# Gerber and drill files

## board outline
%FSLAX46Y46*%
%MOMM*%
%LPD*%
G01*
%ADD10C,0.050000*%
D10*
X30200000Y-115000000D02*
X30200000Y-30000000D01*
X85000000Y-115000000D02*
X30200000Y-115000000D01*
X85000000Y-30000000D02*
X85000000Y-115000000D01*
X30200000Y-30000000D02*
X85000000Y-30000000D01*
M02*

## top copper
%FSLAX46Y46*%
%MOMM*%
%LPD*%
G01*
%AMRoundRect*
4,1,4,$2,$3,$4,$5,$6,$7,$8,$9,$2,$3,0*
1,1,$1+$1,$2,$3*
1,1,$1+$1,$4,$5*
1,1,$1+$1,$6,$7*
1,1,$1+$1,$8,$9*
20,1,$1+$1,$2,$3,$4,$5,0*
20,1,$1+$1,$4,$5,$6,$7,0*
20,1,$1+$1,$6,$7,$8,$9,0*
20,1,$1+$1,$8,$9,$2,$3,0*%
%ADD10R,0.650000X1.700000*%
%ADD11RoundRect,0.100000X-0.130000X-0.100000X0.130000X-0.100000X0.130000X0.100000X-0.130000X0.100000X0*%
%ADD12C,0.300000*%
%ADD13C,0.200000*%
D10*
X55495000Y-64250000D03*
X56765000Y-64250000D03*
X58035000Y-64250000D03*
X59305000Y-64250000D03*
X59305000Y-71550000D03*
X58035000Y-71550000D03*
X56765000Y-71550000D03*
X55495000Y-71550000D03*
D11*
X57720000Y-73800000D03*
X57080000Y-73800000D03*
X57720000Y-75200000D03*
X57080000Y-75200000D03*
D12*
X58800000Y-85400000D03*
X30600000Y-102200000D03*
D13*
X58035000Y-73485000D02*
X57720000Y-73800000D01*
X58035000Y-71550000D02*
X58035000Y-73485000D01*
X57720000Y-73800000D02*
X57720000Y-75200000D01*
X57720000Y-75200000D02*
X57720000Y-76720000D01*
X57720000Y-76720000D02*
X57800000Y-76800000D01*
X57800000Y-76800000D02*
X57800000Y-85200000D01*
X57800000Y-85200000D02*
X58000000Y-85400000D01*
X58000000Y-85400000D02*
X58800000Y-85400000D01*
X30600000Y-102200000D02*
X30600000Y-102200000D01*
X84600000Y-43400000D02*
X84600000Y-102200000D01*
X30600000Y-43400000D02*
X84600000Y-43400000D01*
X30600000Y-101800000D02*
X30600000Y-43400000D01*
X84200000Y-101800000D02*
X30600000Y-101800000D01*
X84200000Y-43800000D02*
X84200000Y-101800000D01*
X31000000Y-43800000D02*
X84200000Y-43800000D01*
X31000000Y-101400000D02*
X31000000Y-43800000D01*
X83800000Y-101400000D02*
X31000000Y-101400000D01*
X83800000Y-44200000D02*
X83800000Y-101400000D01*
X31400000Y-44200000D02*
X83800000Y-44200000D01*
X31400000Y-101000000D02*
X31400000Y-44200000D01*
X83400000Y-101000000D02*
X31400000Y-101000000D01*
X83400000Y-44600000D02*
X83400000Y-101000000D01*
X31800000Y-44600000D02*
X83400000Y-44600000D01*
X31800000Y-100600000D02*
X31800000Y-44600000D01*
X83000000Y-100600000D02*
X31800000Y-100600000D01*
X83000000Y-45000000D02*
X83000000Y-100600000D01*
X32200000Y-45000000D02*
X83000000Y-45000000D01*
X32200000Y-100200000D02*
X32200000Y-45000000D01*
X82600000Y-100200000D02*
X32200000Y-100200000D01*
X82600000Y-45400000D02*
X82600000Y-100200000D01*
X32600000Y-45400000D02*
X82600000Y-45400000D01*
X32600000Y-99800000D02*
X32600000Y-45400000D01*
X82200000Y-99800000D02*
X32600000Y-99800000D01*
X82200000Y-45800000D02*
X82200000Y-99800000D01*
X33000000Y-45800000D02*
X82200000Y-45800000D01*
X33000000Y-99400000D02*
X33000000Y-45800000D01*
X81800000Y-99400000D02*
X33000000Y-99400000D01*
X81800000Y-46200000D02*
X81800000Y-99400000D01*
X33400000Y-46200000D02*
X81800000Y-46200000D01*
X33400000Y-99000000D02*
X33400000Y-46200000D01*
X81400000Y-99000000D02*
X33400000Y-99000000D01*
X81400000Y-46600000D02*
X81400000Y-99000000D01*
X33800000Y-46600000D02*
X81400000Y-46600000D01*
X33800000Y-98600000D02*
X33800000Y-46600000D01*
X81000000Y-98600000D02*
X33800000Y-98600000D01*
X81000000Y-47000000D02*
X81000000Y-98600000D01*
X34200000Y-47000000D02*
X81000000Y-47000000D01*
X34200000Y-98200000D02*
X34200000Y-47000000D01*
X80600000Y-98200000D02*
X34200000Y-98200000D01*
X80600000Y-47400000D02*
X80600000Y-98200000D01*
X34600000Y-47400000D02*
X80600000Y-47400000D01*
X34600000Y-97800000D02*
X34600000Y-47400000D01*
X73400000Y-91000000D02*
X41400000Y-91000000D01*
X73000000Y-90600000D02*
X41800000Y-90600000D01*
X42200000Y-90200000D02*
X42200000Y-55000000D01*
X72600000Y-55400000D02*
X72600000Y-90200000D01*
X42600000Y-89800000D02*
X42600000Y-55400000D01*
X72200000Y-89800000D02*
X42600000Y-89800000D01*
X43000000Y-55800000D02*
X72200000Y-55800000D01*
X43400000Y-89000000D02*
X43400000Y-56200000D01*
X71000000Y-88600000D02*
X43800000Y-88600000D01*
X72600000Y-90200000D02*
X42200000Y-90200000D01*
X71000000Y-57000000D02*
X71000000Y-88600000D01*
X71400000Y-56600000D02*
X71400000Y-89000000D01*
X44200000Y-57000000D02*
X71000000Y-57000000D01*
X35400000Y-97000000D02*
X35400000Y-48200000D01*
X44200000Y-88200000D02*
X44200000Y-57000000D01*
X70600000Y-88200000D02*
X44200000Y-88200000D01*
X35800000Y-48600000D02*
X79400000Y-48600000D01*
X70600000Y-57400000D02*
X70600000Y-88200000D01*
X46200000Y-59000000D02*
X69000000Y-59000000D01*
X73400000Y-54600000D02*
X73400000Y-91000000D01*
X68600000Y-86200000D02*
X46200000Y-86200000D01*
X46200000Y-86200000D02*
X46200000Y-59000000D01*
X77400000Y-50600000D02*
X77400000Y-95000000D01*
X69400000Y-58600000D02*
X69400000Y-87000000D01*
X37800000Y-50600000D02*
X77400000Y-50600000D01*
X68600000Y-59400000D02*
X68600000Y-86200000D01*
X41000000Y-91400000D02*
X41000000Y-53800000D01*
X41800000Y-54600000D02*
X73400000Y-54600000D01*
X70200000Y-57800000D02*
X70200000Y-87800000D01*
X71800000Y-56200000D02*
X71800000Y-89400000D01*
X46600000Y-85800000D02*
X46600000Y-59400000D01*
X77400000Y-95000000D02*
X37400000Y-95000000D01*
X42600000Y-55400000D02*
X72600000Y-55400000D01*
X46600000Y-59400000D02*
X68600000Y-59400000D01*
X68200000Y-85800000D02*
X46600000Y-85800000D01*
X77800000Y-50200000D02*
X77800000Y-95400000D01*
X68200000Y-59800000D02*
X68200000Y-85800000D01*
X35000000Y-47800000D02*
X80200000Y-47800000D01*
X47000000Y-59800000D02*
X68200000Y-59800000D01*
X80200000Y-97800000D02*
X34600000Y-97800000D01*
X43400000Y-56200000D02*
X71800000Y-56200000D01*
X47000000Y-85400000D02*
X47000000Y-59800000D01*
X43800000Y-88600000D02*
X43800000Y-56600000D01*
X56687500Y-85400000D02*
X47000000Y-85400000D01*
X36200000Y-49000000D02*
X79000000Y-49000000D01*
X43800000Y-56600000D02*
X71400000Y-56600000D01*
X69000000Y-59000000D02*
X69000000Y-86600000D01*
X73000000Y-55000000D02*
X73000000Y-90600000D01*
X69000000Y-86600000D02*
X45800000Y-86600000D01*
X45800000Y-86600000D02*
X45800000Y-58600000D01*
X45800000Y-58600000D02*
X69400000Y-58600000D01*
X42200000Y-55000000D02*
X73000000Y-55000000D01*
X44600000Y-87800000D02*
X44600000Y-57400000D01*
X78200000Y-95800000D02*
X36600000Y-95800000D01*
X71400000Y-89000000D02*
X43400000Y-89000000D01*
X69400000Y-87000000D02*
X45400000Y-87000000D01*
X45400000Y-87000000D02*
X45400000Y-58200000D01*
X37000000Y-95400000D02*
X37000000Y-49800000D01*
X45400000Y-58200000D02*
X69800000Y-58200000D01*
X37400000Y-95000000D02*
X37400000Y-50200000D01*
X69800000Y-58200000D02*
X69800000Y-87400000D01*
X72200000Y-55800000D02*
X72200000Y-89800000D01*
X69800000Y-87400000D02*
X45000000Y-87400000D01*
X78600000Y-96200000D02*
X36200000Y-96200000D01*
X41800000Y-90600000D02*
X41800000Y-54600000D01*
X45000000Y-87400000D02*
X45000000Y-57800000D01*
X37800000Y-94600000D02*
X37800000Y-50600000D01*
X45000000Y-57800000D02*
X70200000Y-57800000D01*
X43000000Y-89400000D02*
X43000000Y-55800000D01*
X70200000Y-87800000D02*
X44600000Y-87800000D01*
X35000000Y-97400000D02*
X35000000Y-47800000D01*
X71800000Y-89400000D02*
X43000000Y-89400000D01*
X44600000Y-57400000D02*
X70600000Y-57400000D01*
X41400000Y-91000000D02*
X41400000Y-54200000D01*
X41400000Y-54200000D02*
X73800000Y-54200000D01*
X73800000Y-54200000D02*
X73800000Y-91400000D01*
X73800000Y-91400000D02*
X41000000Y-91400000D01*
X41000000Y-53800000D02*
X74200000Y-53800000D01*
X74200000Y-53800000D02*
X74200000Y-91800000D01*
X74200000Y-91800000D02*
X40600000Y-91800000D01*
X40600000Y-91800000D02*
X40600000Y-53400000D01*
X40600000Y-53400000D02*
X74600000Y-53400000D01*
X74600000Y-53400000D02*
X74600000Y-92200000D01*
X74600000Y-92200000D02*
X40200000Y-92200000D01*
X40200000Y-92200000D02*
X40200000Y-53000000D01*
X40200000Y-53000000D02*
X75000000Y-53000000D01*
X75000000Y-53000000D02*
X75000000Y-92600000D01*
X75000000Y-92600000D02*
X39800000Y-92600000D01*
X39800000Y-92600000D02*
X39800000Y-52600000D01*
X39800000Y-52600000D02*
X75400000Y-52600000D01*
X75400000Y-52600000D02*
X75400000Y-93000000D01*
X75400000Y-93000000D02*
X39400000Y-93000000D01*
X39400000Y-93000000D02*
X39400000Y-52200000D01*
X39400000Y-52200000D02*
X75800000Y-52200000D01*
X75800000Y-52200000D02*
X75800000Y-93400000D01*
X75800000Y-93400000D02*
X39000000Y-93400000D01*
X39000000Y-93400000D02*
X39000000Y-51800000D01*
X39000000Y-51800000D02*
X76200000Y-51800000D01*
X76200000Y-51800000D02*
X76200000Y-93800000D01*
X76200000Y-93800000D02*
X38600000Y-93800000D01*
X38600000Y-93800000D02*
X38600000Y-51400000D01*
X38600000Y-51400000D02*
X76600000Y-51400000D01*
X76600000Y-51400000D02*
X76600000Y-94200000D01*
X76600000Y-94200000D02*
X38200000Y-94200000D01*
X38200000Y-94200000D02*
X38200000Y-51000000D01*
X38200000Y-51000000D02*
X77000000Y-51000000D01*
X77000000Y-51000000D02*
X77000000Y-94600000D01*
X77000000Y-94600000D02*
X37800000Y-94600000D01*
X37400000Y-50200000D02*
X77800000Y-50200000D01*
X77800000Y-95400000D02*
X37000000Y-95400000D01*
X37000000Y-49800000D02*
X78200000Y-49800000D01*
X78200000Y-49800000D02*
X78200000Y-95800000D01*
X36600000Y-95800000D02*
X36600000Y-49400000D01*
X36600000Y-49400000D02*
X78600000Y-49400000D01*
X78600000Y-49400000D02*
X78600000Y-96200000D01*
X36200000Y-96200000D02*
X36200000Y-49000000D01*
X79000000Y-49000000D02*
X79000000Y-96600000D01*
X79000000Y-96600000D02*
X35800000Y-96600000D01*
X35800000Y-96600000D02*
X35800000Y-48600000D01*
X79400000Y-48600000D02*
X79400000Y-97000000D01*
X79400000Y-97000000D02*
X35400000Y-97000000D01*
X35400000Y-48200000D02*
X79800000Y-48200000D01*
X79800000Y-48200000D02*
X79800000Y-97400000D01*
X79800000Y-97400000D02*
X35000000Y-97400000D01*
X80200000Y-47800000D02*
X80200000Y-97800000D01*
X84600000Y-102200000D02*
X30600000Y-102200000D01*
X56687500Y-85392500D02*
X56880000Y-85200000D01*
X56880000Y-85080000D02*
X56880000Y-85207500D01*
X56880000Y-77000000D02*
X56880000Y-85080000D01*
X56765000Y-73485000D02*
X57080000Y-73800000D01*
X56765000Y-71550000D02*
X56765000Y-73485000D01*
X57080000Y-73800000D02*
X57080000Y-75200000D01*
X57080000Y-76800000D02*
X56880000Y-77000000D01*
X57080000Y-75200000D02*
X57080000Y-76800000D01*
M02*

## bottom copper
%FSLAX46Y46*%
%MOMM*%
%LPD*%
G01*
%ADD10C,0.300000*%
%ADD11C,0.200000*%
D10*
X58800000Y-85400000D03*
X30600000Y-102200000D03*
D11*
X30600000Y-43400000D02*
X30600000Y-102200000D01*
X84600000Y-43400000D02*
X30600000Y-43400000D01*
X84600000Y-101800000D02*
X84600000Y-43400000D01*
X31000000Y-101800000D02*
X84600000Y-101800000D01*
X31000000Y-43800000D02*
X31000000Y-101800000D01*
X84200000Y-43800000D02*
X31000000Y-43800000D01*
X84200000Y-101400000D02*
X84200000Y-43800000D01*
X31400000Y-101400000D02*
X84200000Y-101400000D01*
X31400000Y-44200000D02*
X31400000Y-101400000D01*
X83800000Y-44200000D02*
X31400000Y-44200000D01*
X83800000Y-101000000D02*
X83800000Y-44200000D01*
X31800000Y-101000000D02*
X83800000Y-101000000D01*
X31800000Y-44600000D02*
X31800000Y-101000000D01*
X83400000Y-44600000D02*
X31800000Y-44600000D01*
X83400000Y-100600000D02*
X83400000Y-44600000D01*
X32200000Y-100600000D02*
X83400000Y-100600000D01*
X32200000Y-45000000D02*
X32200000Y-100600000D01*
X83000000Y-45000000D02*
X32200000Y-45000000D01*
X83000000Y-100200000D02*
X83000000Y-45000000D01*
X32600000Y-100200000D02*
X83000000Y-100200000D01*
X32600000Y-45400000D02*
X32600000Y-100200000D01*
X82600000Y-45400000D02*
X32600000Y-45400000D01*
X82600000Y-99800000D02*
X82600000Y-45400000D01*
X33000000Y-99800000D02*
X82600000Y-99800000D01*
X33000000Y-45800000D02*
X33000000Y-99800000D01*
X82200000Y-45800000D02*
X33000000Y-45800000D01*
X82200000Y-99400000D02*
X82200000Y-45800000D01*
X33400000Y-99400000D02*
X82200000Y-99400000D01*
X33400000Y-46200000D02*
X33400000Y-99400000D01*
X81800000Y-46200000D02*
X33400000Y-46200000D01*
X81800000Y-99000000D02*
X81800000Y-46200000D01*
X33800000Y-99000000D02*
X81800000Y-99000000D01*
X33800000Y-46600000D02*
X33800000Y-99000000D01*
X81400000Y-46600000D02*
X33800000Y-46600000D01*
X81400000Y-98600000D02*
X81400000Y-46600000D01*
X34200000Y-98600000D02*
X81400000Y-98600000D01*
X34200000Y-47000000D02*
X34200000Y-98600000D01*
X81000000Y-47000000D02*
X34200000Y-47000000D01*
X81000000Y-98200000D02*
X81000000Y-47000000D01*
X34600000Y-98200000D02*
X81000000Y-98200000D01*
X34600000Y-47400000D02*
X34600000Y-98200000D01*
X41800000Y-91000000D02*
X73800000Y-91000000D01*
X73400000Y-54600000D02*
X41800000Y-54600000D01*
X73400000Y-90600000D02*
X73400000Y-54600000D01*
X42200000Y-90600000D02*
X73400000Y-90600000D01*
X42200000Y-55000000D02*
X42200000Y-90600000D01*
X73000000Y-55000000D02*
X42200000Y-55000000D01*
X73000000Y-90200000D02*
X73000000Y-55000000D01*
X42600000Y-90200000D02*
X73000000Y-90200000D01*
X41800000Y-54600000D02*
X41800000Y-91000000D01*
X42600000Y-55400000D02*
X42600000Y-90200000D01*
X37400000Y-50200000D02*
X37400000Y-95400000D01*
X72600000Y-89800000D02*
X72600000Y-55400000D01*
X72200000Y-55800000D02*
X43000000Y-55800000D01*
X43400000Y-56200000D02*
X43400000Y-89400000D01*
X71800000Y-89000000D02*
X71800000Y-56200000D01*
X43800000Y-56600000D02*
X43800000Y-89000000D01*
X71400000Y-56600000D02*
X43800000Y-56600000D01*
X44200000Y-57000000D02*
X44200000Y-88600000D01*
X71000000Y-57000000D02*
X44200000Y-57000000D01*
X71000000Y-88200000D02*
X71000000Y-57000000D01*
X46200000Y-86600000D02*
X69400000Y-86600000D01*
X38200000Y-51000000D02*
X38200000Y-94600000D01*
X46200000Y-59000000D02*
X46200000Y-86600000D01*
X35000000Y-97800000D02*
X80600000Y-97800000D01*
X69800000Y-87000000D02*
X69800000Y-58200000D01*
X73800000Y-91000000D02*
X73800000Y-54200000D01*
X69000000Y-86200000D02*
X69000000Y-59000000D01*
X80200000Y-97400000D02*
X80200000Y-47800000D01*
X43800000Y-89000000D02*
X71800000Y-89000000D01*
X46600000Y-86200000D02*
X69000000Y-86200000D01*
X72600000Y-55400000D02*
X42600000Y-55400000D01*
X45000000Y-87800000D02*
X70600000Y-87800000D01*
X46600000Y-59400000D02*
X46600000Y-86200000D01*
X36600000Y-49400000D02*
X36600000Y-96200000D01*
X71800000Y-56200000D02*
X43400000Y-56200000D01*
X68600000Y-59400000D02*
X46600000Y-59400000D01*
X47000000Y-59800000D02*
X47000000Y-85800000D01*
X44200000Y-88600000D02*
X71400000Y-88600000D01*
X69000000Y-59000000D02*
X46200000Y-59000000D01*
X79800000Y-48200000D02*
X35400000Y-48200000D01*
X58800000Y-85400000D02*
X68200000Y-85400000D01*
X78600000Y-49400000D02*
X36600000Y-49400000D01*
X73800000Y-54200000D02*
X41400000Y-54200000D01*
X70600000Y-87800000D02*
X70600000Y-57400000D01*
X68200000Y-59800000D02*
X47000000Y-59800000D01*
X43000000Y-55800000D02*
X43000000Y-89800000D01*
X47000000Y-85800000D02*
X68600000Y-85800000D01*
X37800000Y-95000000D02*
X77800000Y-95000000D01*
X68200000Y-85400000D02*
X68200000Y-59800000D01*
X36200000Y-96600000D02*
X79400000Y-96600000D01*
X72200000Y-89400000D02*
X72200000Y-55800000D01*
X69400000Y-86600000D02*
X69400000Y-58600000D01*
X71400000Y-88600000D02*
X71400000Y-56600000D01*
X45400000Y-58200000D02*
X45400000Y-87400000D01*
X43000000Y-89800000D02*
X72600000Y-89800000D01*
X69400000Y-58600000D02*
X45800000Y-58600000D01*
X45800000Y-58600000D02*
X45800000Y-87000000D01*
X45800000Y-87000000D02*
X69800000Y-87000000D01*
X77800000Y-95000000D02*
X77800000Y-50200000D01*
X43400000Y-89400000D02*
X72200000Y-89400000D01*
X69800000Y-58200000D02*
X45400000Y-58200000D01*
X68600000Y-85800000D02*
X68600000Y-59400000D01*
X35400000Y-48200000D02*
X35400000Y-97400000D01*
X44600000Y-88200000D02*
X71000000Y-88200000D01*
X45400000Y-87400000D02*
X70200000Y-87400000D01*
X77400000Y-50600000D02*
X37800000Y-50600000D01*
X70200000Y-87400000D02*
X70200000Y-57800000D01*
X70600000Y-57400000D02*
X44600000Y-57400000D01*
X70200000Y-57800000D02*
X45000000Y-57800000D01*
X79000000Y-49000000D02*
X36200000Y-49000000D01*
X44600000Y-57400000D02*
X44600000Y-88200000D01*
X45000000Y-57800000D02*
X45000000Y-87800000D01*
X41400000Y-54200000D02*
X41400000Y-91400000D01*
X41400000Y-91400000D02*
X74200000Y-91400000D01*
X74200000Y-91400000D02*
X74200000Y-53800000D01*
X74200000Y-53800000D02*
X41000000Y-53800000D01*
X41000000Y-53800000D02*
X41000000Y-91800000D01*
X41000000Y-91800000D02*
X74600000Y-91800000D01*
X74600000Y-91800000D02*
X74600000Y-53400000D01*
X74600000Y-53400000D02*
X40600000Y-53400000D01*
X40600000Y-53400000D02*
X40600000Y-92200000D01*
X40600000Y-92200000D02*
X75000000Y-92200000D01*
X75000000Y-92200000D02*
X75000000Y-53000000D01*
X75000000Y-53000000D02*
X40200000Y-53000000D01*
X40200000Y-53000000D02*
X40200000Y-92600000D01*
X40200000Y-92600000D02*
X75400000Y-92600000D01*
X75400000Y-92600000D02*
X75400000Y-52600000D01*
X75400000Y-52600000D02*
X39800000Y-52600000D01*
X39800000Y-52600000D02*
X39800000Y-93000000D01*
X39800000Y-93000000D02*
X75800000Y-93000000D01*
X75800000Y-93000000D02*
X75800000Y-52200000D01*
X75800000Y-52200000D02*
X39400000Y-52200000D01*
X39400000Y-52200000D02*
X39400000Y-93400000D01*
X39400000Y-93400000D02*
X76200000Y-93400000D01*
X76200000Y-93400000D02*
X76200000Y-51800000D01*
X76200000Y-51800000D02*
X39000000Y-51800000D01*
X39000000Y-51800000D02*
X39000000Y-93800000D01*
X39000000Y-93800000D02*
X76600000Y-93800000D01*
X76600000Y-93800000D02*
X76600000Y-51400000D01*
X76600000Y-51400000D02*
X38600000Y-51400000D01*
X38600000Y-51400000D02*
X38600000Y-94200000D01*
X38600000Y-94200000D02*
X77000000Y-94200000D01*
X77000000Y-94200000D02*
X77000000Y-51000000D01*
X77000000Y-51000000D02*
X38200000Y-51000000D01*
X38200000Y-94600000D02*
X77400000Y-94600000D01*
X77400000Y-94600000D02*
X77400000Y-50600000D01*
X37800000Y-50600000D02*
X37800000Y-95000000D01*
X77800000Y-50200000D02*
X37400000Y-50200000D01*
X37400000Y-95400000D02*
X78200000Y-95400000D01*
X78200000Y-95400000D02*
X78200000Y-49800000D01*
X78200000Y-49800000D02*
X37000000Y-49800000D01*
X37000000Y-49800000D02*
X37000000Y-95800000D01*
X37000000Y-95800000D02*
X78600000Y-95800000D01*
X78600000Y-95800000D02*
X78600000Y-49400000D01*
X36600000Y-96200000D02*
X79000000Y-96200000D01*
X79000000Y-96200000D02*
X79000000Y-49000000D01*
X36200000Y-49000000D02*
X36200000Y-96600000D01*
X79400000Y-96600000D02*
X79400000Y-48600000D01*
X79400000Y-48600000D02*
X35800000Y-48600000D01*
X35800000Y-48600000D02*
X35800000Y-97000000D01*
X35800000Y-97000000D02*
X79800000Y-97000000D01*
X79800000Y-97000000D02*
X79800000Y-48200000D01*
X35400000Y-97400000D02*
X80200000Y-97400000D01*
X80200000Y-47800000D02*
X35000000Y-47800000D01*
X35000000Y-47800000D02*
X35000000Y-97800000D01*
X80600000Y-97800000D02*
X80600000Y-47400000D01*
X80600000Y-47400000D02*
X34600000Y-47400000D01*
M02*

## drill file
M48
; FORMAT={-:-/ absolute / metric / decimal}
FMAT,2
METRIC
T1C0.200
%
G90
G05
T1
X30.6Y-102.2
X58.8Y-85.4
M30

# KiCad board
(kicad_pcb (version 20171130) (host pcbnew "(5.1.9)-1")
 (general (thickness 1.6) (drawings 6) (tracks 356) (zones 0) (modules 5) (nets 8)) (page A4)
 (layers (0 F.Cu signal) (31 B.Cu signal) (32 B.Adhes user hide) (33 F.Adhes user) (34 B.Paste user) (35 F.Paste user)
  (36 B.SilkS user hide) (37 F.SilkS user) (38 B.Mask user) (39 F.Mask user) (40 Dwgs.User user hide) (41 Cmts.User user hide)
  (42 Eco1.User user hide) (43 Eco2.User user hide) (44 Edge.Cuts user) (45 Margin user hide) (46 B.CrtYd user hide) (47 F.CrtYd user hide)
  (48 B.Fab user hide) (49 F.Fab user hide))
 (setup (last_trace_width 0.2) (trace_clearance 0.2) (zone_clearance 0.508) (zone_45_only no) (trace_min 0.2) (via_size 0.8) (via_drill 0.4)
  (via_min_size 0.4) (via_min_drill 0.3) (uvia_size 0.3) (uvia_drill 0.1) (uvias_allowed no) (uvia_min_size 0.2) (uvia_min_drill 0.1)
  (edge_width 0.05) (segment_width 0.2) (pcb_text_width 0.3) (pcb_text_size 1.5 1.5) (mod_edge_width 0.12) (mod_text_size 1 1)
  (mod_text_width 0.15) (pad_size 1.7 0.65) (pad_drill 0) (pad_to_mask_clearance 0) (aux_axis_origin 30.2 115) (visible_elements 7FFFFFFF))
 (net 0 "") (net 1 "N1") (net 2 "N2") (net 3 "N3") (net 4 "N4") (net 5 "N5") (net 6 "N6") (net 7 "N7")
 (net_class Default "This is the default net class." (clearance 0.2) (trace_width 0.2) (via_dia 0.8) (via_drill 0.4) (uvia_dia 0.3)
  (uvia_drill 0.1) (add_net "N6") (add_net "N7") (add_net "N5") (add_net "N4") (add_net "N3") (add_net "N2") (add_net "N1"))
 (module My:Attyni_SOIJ (layer F.Cu) (at 57.4 67.9 90)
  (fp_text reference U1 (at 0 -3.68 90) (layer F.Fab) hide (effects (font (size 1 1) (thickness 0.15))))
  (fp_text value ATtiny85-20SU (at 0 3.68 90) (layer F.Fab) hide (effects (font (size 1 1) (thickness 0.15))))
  (pad 8 smd rect (at 3.65 -1.905 90) (size 1.7 0.65) (layers F.Cu F.Paste F.Mask) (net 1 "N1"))
  (pad 7 smd rect (at 3.65 -0.635 90) (size 1.7 0.65) (layers F.Cu F.Paste F.Mask) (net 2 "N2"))
  (pad 6 smd rect (at 3.65 0.635 90) (size 1.7 0.65) (layers F.Cu F.Paste F.Mask) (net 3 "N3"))
  (pad 5 smd rect (at 3.65 1.905 90) (size 1.7 0.65) (layers F.Cu F.Paste F.Mask) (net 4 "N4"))
  (pad 4 smd rect (at -3.65 1.905 90) (size 1.7 0.65) (layers F.Cu F.Paste F.Mask) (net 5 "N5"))
  (pad 3 smd rect (at -3.65 0.635 90) (size 1.7 0.65) (layers F.Cu F.Paste F.Mask) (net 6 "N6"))
  (pad 2 smd rect (at -3.65 -0.635 90) (size 1.7 0.65) (layers F.Cu F.Paste F.Mask) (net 6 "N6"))
  (pad 1 smd rect (at -3.65 -1.905 90) (size 1.7 0.65) (layers F.Cu F.Paste F.Mask) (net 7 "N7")))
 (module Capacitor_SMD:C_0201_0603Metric (layer F.Cu) (at 57.4 73.8)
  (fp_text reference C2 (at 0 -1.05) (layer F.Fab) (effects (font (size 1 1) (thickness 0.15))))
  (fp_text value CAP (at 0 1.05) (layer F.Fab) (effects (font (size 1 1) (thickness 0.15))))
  (pad 2 smd roundrect (at 0.32 0) (size 0.46 0.4) (layers F.Cu F.Mask) (roundrect_rratio 0.25) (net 6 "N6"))
  (pad 1 smd roundrect (at -0.32 0) (size 0.46 0.4) (layers F.Cu F.Mask) (roundrect_rratio 0.25) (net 6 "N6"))
  (pad "" smd roundrect (at 0.345 0) (size 0.318 0.36) (layers F.Paste) (roundrect_rratio 0.25))
  (pad "" smd roundrect (at -0.345 0) (size 0.318 0.36) (layers F.Paste) (roundrect_rratio 0.25)))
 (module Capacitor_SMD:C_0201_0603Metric (layer F.Cu) (at 57.4 75.2)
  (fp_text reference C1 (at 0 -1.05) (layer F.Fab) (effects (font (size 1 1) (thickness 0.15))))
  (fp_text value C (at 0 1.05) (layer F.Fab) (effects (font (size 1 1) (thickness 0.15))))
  (pad 2 smd roundrect (at 0.32 0) (size 0.46 0.4) (layers F.Cu F.Mask) (roundrect_rratio 0.25) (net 6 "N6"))
  (pad 1 smd roundrect (at -0.32 0) (size 0.46 0.4) (layers F.Cu F.Mask) (roundrect_rratio 0.25) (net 6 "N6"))
  (pad "" smd roundrect (at 0.345 0) (size 0.318 0.36) (layers F.Paste) (roundrect_rratio 0.25))
  (pad "" smd roundrect (at -0.345 0) (size 0.318 0.36) (layers F.Paste) (roundrect_rratio 0.25)))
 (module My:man (layer F.Cu) (at 51.6 77.8)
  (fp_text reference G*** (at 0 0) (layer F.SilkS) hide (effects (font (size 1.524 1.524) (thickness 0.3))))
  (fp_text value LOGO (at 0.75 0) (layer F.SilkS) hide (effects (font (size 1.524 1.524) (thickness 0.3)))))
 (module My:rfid (layer B.Cu) (at 58.4 70.6 180)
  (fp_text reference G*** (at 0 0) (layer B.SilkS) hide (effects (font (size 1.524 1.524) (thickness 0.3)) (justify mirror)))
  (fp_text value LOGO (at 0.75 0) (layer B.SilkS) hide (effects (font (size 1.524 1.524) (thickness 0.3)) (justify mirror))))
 (gr_line (start 30.2 115) (end 30.2 30) (layer Edge.Cuts) (width 0.05))
 (gr_line (start 85 115) (end 30.2 115) (layer Edge.Cuts) (width 0.05))
 (gr_line (start 85 30) (end 85 115) (layer Edge.Cuts) (width 0.05))
 (gr_line (start 30.2 30) (end 85 30) (layer Edge.Cuts) (width 0.05))
 (segment (start 58.035 73.485) (end 57.72 73.8) (width 0.2) (layer F.Cu) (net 6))
 (segment (start 58.035 71.55) (end 58.035 73.485) (width 0.2) (layer F.Cu) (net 6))
 (segment (start 57.72 73.8) (end 57.72 75.2) (width 0.2) (layer F.Cu) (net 6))
 (segment (start 57.72 75.2) (end 57.72 76.72) (width 0.2) (layer F.Cu) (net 6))
 (segment (start 57.72 76.72) (end 57.8 76.8) (width 0.2) (layer F.Cu) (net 6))
 (segment (start 57.8 76.8) (end 57.8 85.2) (width 0.2) (layer F.Cu) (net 6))
 (segment (start 57.8 85.2) (end 58 85.4) (width 0.2) (layer F.Cu) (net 6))
 (segment (start 58 85.4) (end 58.8 85.4) (width 0.2) (layer F.Cu) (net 6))
 (via (at 58.8 85.4) (size 0.3) (drill 0.2) (layers F.Cu B.Cu) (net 6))
 (segment (start 30.6 102.2) (end 30.6 102.2) (width 0.2) (layer F.Cu) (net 6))
 (segment (start 84.6 43.4) (end 84.6 102.2) (width 0.2) (layer F.Cu) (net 6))
 (segment (start 30.6 43.4) (end 84.6 43.4) (width 0.2) (layer F.Cu) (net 6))
 (segment (start 30.6 101.8) (end 30.6 43.4) (width 0.2) (layer F.Cu) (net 6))
 (segment (start 84.2 101.8) (end 30.6 101.8) (width 0.2) (layer F.Cu) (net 6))
 (segment (start 84.2 43.8) (end 84.2 101.8) (width 0.2) (layer F.Cu) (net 6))
 (segment (start 31 43.8) (end 84.2 43.8) (width 0.2) (layer F.Cu) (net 6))
 (segment (start 31 101.4) (end 31 43.8) (width 0.2) (layer F.Cu) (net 6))
 (segment (start 83.8 101.4) (end 31 101.4) (width 0.2) (layer F.Cu) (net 6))
 (segment (start 83.8 44.2) (end 83.8 101.4) (width 0.2) (layer F.Cu) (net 6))
 (segment (start 31.4 44.2) (end 83.8 44.2) (width 0.2) (layer F.Cu) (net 6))
 (segment (start 31.4 101) (end 31.4 44.2) (width 0.2) (layer F.Cu) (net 6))
 (segment (start 83.4 101) (end 31.4 101) (width 0.2) (layer F.Cu) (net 6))
 (segment (start 83.4 44.6) (end 83.4 101) (width 0.2) (layer F.Cu) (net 6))
 (segment (start 31.8 44.6) (end 83.4 44.6) (width 0.2) (layer F.Cu) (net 6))
 (segment (start 31.8 100.6) (end 31.8 44.6) (width 0.2) (layer F.Cu) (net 6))
 (segment (start 83 100.6) (end 31.8 100.6) (width 0.2) (layer F.Cu) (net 6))
 (segment (start 83 45) (end 83 100.6) (width 0.2) (layer F.Cu) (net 6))
 (segment (start 32.2 45) (end 83 45) (width 0.2) (layer F.Cu) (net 6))
 (segment (start 32.2 100.2) (end 32.2 45) (width 0.2) (layer F.Cu) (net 6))
 (segment (start 82.6 100.2) (end 32.2 100.2) (width 0.2) (layer F.Cu) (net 6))
 (segment (start 82.6 45.4) (end 82.6 100.2) (width 0.2) (layer F.Cu) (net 6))
 (segment (start 32.6 45.4) (end 82.6 45.4) (width 0.2) (layer F.Cu) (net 6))
 (segment (start 32.6 99.8) (end 32.6 45.4) (width 0.2) (layer F.Cu) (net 6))
 (segment (start 82.2 99.8) (end 32.6 99.8) (width 0.2) (layer F.Cu) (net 6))
 (segment (start 82.2 45.8) (end 82.2 99.8) (width 0.2) (layer F.Cu) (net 6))
 (segment (start 33 45.8) (end 82.2 45.8) (width 0.2) (layer F.Cu) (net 6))
 (segment (start 33 99.4) (end 33 45.8) (width 0.2) (layer F.Cu) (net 6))
 (segment (start 81.8 99.4) (end 33 99.4) (width 0.2) (layer F.Cu) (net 6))
 (segment (start 81.8 46.2) (end 81.8 99.4) (width 0.2) (layer F.Cu) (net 6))
 (segment (start 33.4 46.2) (end 81.8 46.2) (width 0.2) (layer F.Cu) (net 6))
 (segment (start 33.4 99) (end 33.4 46.2) (width 0.2) (layer F.Cu) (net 6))
 (segment (start 81.4 99) (end 33.4 99) (width 0.2) (layer F.Cu) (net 6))
 (segment (start 81.4 46.6) (end 81.4 99) (width 0.2) (layer F.Cu) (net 6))
 (segment (start 33.8 46.6) (end 81.4 46.6) (width 0.2) (layer F.Cu) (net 6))
 (segment (start 33.8 98.6) (end 33.8 46.6) (width 0.2) (layer F.Cu) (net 6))
 (segment (start 81 98.6) (end 33.8 98.6) (width 0.2) (layer F.Cu) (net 6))
 (segment (start 81 47) (end 81 98.6) (width 0.2) (layer F.Cu) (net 6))
 (segment (start 34.2 47) (end 81 47) (width 0.2) (layer F.Cu) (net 6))
 (segment (start 34.2 98.2) (end 34.2 47) (width 0.2) (layer F.Cu) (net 6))
 (segment (start 80.6 98.2) (end 34.2 98.2) (width 0.2) (layer F.Cu) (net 6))
 (segment (start 80.6 47.4) (end 80.6 98.2) (width 0.2) (layer F.Cu) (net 6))
 (segment (start 34.6 47.4) (end 80.6 47.4) (width 0.2) (layer F.Cu) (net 6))
 (segment (start 34.6 97.8) (end 34.6 47.4) (width 0.2) (layer F.Cu) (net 6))
 (segment (start 73.4 91) (end 41.4 91) (width 0.2) (layer F.Cu) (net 6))
 (segment (start 73 90.6) (end 41.8 90.6) (width 0.2) (layer F.Cu) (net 6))
 (segment (start 42.2 90.2) (end 42.2 55) (width 0.2) (layer F.Cu) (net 6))
 (segment (start 72.6 55.4) (end 72.6 90.2) (width 0.2) (layer F.Cu) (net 6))
 (segment (start 42.6 89.8) (end 42.6 55.4) (width 0.2) (layer F.Cu) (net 6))
 (segment (start 72.2 89.8) (end 42.6 89.8) (width 0.2) (layer F.Cu) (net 6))
 (segment (start 43 55.8) (end 72.2 55.8) (width 0.2) (layer F.Cu) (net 6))
 (segment (start 43.4 89) (end 43.4 56.2) (width 0.2) (layer F.Cu) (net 6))
 (segment (start 71 88.6) (end 43.8 88.6) (width 0.2) (layer F.Cu) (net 6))
 (segment (start 72.6 90.2) (end 42.2 90.2) (width 0.2) (layer F.Cu) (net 6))
 (segment (start 71 57) (end 71 88.6) (width 0.2) (layer F.Cu) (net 6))
 (segment (start 71.4 56.6) (end 71.4 89) (width 0.2) (layer F.Cu) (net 6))
 (segment (start 44.2 57) (end 71 57) (width 0.2) (layer F.Cu) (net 6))
 (segment (start 35.4 97) (end 35.4 48.2) (width 0.2) (layer F.Cu) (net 6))
 (segment (start 44.2 88.2) (end 44.2 57) (width 0.2) (layer F.Cu) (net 6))
 (segment (start 70.6 88.2) (end 44.2 88.2) (width 0.2) (layer F.Cu) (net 6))
 (segment (start 35.8 48.6) (end 79.4 48.6) (width 0.2) (layer F.Cu) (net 6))
 (segment (start 70.6 57.4) (end 70.6 88.2) (width 0.2) (layer F.Cu) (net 6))
 (segment (start 46.2 59) (end 69 59) (width 0.2) (layer F.Cu) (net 6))
 (segment (start 73.4 54.6) (end 73.4 91) (width 0.2) (layer F.Cu) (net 6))
 (segment (start 68.6 86.2) (end 46.2 86.2) (width 0.2) (layer F.Cu) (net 6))
 (segment (start 46.2 86.2) (end 46.2 59) (width 0.2) (layer F.Cu) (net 6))
 (segment (start 77.4 50.6) (end 77.4 95) (width 0.2) (layer F.Cu) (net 6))
 (segment (start 69.4 58.6) (end 69.4 87) (width 0.2) (layer F.Cu) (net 6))
 (segment (start 37.8 50.6) (end 77.4 50.6) (width 0.2) (layer F.Cu) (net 6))
 (segment (start 68.6 59.4) (end 68.6 86.2) (width 0.2) (layer F.Cu) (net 6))
 (segment (start 41 91.4) (end 41 53.8) (width 0.2) (layer F.Cu) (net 6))
 (segment (start 41.8 54.6) (end 73.4 54.6) (width 0.2) (layer F.Cu) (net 6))
 (segment (start 70.2 57.8) (end 70.2 87.8) (width 0.2) (layer F.Cu) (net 6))
 (segment (start 71.8 56.2) (end 71.8 89.4) (width 0.2) (layer F.Cu) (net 6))
 (segment (start 46.6 85.8) (end 46.6 59.4) (width 0.2) (layer F.Cu) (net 6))
 (segment (start 77.4 95) (end 37.4 95) (width 0.2) (layer F.Cu) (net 6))
 (segment (start 42.6 55.4) (end 72.6 55.4) (width 0.2) (layer F.Cu) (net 6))
 (segment (start 46.6 59.4) (end 68.6 59.4) (width 0.2) (layer F.Cu) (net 6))
 (segment (start 68.2 85.8) (end 46.6 85.8) (width 0.2) (layer F.Cu) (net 6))
 (segment (start 77.8 50.2) (end 77.8 95.4) (width 0.2) (layer F.Cu) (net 6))
 (segment (start 68.2 59.8) (end 68.2 85.8) (width 0.2) (layer F.Cu) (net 6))
 (segment (start 35 47.8) (end 80.2 47.8) (width 0.2) (layer F.Cu) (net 6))
 (segment (start 47 59.8) (end 68.2 59.8) (width 0.2) (layer F.Cu) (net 6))
 (segment (start 80.2 97.8) (end 34.6 97.8) (width 0.2) (layer F.Cu) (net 6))
 (segment (start 43.4 56.2) (end 71.8 56.2) (width 0.2) (layer F.Cu) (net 6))
 (segment (start 47 85.4) (end 47 59.8) (width 0.2) (layer F.Cu) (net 6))
 (segment (start 43.8 88.6) (end 43.8 56.6) (width 0.2) (layer F.Cu) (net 6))
 (segment (start 56.6875 85.4) (end 47 85.4) (width 0.2) (layer F.Cu) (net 6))
 (segment (start 36.2 49) (end 79 49) (width 0.2) (layer F.Cu) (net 6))
 (segment (start 43.8 56.6) (end 71.4 56.6) (width 0.2) (layer F.Cu) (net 6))
 (segment (start 69 59) (end 69 86.6) (width 0.2) (layer F.Cu) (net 6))
 (segment (start 73 55) (end 73 90.6) (width 0.2) (layer F.Cu) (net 6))
 (segment (start 69 86.6) (end 45.8 86.6) (width 0.2) (layer F.Cu) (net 6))
 (segment (start 45.8 86.6) (end 45.8 58.6) (width 0.2) (layer F.Cu) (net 6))
 (segment (start 45.8 58.6) (end 69.4 58.6) (width 0.2) (layer F.Cu) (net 6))
 (segment (start 42.2 55) (end 73 55) (width 0.2) (layer F.Cu) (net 6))
 (segment (start 44.6 87.8) (end 44.6 57.4) (width 0.2) (layer F.Cu) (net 6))
 (segment (start 78.2 95.8) (end 36.6 95.8) (width 0.2) (layer F.Cu) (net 6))
 (segment (start 71.4 89) (end 43.4 89) (width 0.2) (layer F.Cu) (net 6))
 (segment (start 69.4 87) (end 45.4 87) (width 0.2) (layer F.Cu) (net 6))
 (segment (start 45.4 87) (end 45.4 58.2) (width 0.2) (layer F.Cu) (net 6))
 (segment (start 37 95.4) (end 37 49.8) (width 0.2) (layer F.Cu) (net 6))
 (segment (start 45.4 58.2) (end 69.8 58.2) (width 0.2) (layer F.Cu) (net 6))
 (segment (start 37.4 95) (end 37.4 50.2) (width 0.2) (layer F.Cu) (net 6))
 (segment (start 69.8 58.2) (end 69.8 87.4) (width 0.2) (layer F.Cu) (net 6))
 (segment (start 72.2 55.8) (end 72.2 89.8) (width 0.2) (layer F.Cu) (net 6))
 (segment (start 69.8 87.4) (end 45 87.4) (width 0.2) (layer F.Cu) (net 6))
 (segment (start 78.6 96.2) (end 36.2 96.2) (width 0.2) (layer F.Cu) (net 6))
 (segment (start 41.8 90.6) (end 41.8 54.6) (width 0.2) (layer F.Cu) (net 6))
 (segment (start 45 87.4) (end 45 57.8) (width 0.2) (layer F.Cu) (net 6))
 (segment (start 37.8 94.6) (end 37.8 50.6) (width 0.2) (layer F.Cu) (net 6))
 (segment (start 45 57.8) (end 70.2 57.8) (width 0.2) (layer F.Cu) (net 6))
 (segment (start 43 89.4) (end 43 55.8) (width 0.2) (layer F.Cu) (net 6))
 (segment (start 70.2 87.8) (end 44.6 87.8) (width 0.2) (layer F.Cu) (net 6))
 (segment (start 35 97.4) (end 35 47.8) (width 0.2) (layer F.Cu) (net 6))
 (segment (start 71.8 89.4) (end 43 89.4) (width 0.2) (layer F.Cu) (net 6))
 (segment (start 44.6 57.4) (end 70.6 57.4) (width 0.2) (layer F.Cu) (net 6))
 (segment (start 41.4 91) (end 41.4 54.2) (width 0.2) (layer F.Cu) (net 6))
 (segment (start 41.4 54.2) (end 73.8 54.2) (width 0.2) (layer F.Cu) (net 6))
 (segment (start 73.8 54.2) (end 73.8 91.4) (width 0.2) (layer F.Cu) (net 6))
 (segment (start 73.8 91.4) (end 41 91.4) (width 0.2) (layer F.Cu) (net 6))
 (segment (start 41 53.8) (end 74.2 53.8) (width 0.2) (layer F.Cu) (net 6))
 (segment (start 74.2 53.8) (end 74.2 91.8) (width 0.2) (layer F.Cu) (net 6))
 (segment (start 74.2 91.8) (end 40.6 91.8) (width 0.2) (layer F.Cu) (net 6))
 (segment (start 40.6 91.8) (end 40.6 53.4) (width 0.2) (layer F.Cu) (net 6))
 (segment (start 40.6 53.4) (end 74.6 53.4) (width 0.2) (layer F.Cu) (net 6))
 (segment (start 74.6 53.4) (end 74.6 92.2) (width 0.2) (layer F.Cu) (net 6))
 (segment (start 74.6 92.2) (end 40.2 92.2) (width 0.2) (layer F.Cu) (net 6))
 (segment (start 40.2 92.2) (end 40.2 53) (width 0.2) (layer F.Cu) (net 6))
 (segment (start 40.2 53) (end 75 53) (width 0.2) (layer F.Cu) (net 6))
 (segment (start 75 53) (end 75 92.6) (width 0.2) (layer F.Cu) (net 6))
 (segment (start 75 92.6) (end 39.8 92.6) (width 0.2) (layer F.Cu) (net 6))
 (segment (start 39.8 92.6) (end 39.8 52.6) (width 0.2) (layer F.Cu) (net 6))
 (segment (start 39.8 52.6) (end 75.4 52.6) (width 0.2) (layer F.Cu) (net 6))
 (segment (start 75.4 52.6) (end 75.4 93) (width 0.2) (layer F.Cu) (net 6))
 (segment (start 75.4 93) (end 39.4 93) (width 0.2) (layer F.Cu) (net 6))
 (segment (start 39.4 93) (end 39.4 52.2) (width 0.2) (layer F.Cu) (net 6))
 (segment (start 39.4 52.2) (end 75.8 52.2) (width 0.2) (layer F.Cu) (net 6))
 (segment (start 75.8 52.2) (end 75.8 93.4) (width 0.2) (layer F.Cu) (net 6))
 (segment (start 75.8 93.4) (end 39 93.4) (width 0.2) (layer F.Cu) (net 6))
 (segment (start 39 93.4) (end 39 51.8) (width 0.2) (layer F.Cu) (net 6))
 (segment (start 39 51.8) (end 76.2 51.8) (width 0.2) (layer F.Cu) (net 6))
 (segment (start 76.2 51.8) (end 76.2 93.8) (width 0.2) (layer F.Cu) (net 6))
 (segment (start 76.2 93.8) (end 38.6 93.8) (width 0.2) (layer F.Cu) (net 6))
 (segment (start 38.6 93.8) (end 38.6 51.4) (width 0.2) (layer F.Cu) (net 6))
 (segment (start 38.6 51.4) (end 76.6 51.4) (width 0.2) (layer F.Cu) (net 6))
 (segment (start 76.6 51.4) (end 76.6 94.2) (width 0.2) (layer F.Cu) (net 6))
 (segment (start 76.6 94.2) (end 38.2 94.2) (width 0.2) (layer F.Cu) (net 6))
 (segment (start 38.2 94.2) (end 38.2 51) (width 0.2) (layer F.Cu) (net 6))
 (segment (start 38.2 51) (end 77 51) (width 0.2) (layer F.Cu) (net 6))
 (segment (start 77 51) (end 77 94.6) (width 0.2) (layer F.Cu) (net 6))
 (segment (start 77 94.6) (end 37.8 94.6) (width 0.2) (layer F.Cu) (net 6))
 (segment (start 37.4 50.2) (end 77.8 50.2) (width 0.2) (layer F.Cu) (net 6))
 (segment (start 77.8 95.4) (end 37 95.4) (width 0.2) (layer F.Cu) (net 6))
 (segment (start 37 49.8) (end 78.2 49.8) (width 0.2) (layer F.Cu) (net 6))
 (segment (start 78.2 49.8) (end 78.2 95.8) (width 0.2) (layer F.Cu) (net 6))
 (segment (start 36.6 95.8) (end 36.6 49.4) (width 0.2) (layer F.Cu) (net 6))
 (segment (start 36.6 49.4) (end 78.6 49.4) (width 0.2) (layer F.Cu) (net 6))
 (segment (start 78.6 49.4) (end 78.6 96.2) (width 0.2) (layer F.Cu) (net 6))
 (segment (start 36.2 96.2) (end 36.2 49) (width 0.2) (layer F.Cu) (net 6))
 (segment (start 79 49) (end 79 96.6) (width 0.2) (layer F.Cu) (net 6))
 (segment (start 79 96.6) (end 35.8 96.6) (width 0.2) (layer F.Cu) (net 6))
 (segment (start 35.8 96.6) (end 35.8 48.6) (width 0.2) (layer F.Cu) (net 6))
 (segment (start 79.4 48.6) (end 79.4 97) (width 0.2) (layer F.Cu) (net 6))
 (segment (start 79.4 97) (end 35.4 97) (width 0.2) (layer F.Cu) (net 6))
 (segment (start 35.4 48.2) (end 79.8 48.2) (width 0.2) (layer F.Cu) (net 6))
 (segment (start 79.8 48.2) (end 79.8 97.4) (width 0.2) (layer F.Cu) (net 6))
 (segment (start 79.8 97.4) (end 35 97.4) (width 0.2) (layer F.Cu) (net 6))
 (segment (start 80.2 47.8) (end 80.2 97.8) (width 0.2) (layer F.Cu) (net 6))
 (segment (start 84.6 102.2) (end 30.6 102.2) (width 0.2) (layer F.Cu) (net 6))
 (segment (start 56.6875 85.3925) (end 56.88 85.2) (width 0.2) (layer F.Cu) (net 6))
 (segment (start 56.88 85.08) (end 56.88 85.2075) (width 0.2) (layer F.Cu) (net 6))
 (segment (start 56.88 77) (end 56.88 85.08) (width 0.2) (layer F.Cu) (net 6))
 (segment (start 56.765 73.485) (end 57.08 73.8) (width 0.2) (layer F.Cu) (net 6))
 (segment (start 56.765 71.55) (end 56.765 73.485) (width 0.2) (layer F.Cu) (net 6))
 (segment (start 57.08 73.8) (end 57.08 75.2) (width 0.2) (layer F.Cu) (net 6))
 (segment (start 57.08 76.8) (end 56.88 77) (width 0.2) (layer F.Cu) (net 6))
 (segment (start 57.08 75.2) (end 57.08 76.8) (width 0.2) (layer F.Cu) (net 6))
 (segment (start 30.6 43.4) (end 30.6 102.2) (width 0.2) (layer B.Cu) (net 6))
 (segment (start 84.6 43.4) (end 30.6 43.4) (width 0.2) (layer B.Cu) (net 6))
 (segment (start 84.6 101.8) (end 84.6 43.4) (width 0.2) (layer B.Cu) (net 6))
 (segment (start 31 101.8) (end 84.6 101.8) (width 0.2) (layer B.Cu) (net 6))
 (segment (start 31 43.8) (end 31 101.8) (width 0.2) (layer B.Cu) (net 6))
 (segment (start 84.2 43.8) (end 31 43.8) (width 0.2) (layer B.Cu) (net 6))
 (segment (start 84.2 101.4) (end 84.2 43.8) (width 0.2) (layer B.Cu) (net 6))
 (segment (start 31.4 101.4) (end 84.2 101.4) (width 0.2) (layer B.Cu) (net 6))
 (segment (start 31.4 44.2) (end 31.4 101.4) (width 0.2) (layer B.Cu) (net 6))
 (segment (start 83.8 44.2) (end 31.4 44.2) (width 0.2) (layer B.Cu) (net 6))
 (segment (start 83.8 101) (end 83.8 44.2) (width 0.2) (layer B.Cu) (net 6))
 (segment (start 31.8 101) (end 83.8 101) (width 0.2) (layer B.Cu) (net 6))
 (segment (start 31.8 44.6) (end 31.8 101) (width 0.2) (layer B.Cu) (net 6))
 (segment (start 83.4 44.6) (end 31.8 44.6) (width 0.2) (layer B.Cu) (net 6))
 (segment (start 83.4 100.6) (end 83.4 44.6) (width 0.2) (layer B.Cu) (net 6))
 (segment (start 32.2 100.6) (end 83.4 100.6) (width 0.2) (layer B.Cu) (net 6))
 (segment (start 32.2 45) (end 32.2 100.6) (width 0.2) (layer B.Cu) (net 6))
 (segment (start 83 45) (end 32.2 45) (width 0.2) (layer B.Cu) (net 6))
 (segment (start 83 100.2) (end 83 45) (width 0.2) (layer B.Cu) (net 6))
 (segment (start 32.6 100.2) (end 83 100.2) (width 0.2) (layer B.Cu) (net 6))
 (segment (start 32.6 45.4) (end 32.6 100.2) (width 0.2) (layer B.Cu) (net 6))
 (segment (start 82.6 45.4) (end 32.6 45.4) (width 0.2) (layer B.Cu) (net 6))
 (segment (start 82.6 99.8) (end 82.6 45.4) (width 0.2) (layer B.Cu) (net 6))
 (segment (start 33 99.8) (end 82.6 99.8) (width 0.2) (layer B.Cu) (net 6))
 (segment (start 33 45.8) (end 33 99.8) (width 0.2) (layer B.Cu) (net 6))
 (segment (start 82.2 45.8) (end 33 45.8) (width 0.2) (layer B.Cu) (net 6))
 (segment (start 82.2 99.4) (end 82.2 45.8) (width 0.2) (layer B.Cu) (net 6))
 (segment (start 33.4 99.4) (end 82.2 99.4) (width 0.2) (layer B.Cu) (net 6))
 (segment (start 33.4 46.2) (end 33.4 99.4) (width 0.2) (layer B.Cu) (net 6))
 (segment (start 81.8 46.2) (end 33.4 46.2) (width 0.2) (layer B.Cu) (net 6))
 (segment (start 81.8 99) (end 81.8 46.2) (width 0.2) (layer B.Cu) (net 6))
 (segment (start 33.8 99) (end 81.8 99) (width 0.2) (layer B.Cu) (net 6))
 (segment (start 33.8 46.6) (end 33.8 99) (width 0.2) (layer B.Cu) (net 6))
 (segment (start 81.4 46.6) (end 33.8 46.6) (width 0.2) (layer B.Cu) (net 6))
 (segment (start 81.4 98.6) (end 81.4 46.6) (width 0.2) (layer B.Cu) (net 6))
 (segment (start 34.2 98.6) (end 81.4 98.6) (width 0.2) (layer B.Cu) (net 6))
 (segment (start 34.2 47) (end 34.2 98.6) (width 0.2) (layer B.Cu) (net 6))
 (segment (start 81 47) (end 34.2 47) (width 0.2) (layer B.Cu) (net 6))
 (segment (start 81 98.2) (end 81 47) (width 0.2) (layer B.Cu) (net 6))
 (segment (start 34.6 98.2) (end 81 98.2) (width 0.2) (layer B.Cu) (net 6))
 (segment (start 34.6 47.4) (end 34.6 98.2) (width 0.2) (layer B.Cu) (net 6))
 (segment (start 41.8 91) (end 73.8 91) (width 0.2) (layer B.Cu) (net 6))
 (segment (start 73.4 54.6) (end 41.8 54.6) (width 0.2) (layer B.Cu) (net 6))
 (segment (start 73.4 90.6) (end 73.4 54.6) (width 0.2) (layer B.Cu) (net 6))
 (segment (start 42.2 90.6) (end 73.4 90.6) (width 0.2) (layer B.Cu) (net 6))
 (segment (start 42.2 55) (end 42.2 90.6) (width 0.2) (layer B.Cu) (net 6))
 (segment (start 73 55) (end 42.2 55) (width 0.2) (layer B.Cu) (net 6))
 (segment (start 73 90.2) (end 73 55) (width 0.2) (layer B.Cu) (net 6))
 (segment (start 42.6 90.2) (end 73 90.2) (width 0.2) (layer B.Cu) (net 6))
 (segment (start 41.8 54.6) (end 41.8 91) (width 0.2) (layer B.Cu) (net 6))
 (segment (start 42.6 55.4) (end 42.6 90.2) (width 0.2) (layer B.Cu) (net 6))
 (segment (start 37.4 50.2) (end 37.4 95.4) (width 0.2) (layer B.Cu) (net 6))
 (segment (start 72.6 89.8) (end 72.6 55.4) (width 0.2) (layer B.Cu) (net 6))
 (segment (start 72.2 55.8) (end 43 55.8) (width 0.2) (layer B.Cu) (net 6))
 (segment (start 43.4 56.2) (end 43.4 89.4) (width 0.2) (layer B.Cu) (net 6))
 (segment (start 71.8 89) (end 71.8 56.2) (width 0.2) (layer B.Cu) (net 6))
 (segment (start 43.8 56.6) (end 43.8 89) (width 0.2) (layer B.Cu) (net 6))
 (segment (start 71.4 56.6) (end 43.8 56.6) (width 0.2) (layer B.Cu) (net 6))
 (segment (start 44.2 57) (end 44.2 88.6) (width 0.2) (layer B.Cu) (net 6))
 (segment (start 71 57) (end 44.2 57) (width 0.2) (layer B.Cu) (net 6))
 (segment (start 71 88.2) (end 71 57) (width 0.2) (layer B.Cu) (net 6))
 (segment (start 46.2 86.6) (end 69.4 86.6) (width 0.2) (layer B.Cu) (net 6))
 (segment (start 38.2 51) (end 38.2 94.6) (width 0.2) (layer B.Cu) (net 6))
 (segment (start 46.2 59) (end 46.2 86.6) (width 0.2) (layer B.Cu) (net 6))
 (segment (start 35 97.8) (end 80.6 97.8) (width 0.2) (layer B.Cu) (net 6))
 (segment (start 69.8 87) (end 69.8 58.2) (width 0.2) (layer B.Cu) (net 6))
 (segment (start 73.8 91) (end 73.8 54.2) (width 0.2) (layer B.Cu) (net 6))
 (segment (start 69 86.2) (end 69 59) (width 0.2) (layer B.Cu) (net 6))
 (segment (start 80.2 97.4) (end 80.2 47.8) (width 0.2) (layer B.Cu) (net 6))
 (segment (start 43.8 89) (end 71.8 89) (width 0.2) (layer B.Cu) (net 6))
 (segment (start 46.6 86.2) (end 69 86.2) (width 0.2) (layer B.Cu) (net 6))
 (segment (start 72.6 55.4) (end 42.6 55.4) (width 0.2) (layer B.Cu) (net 6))
 (segment (start 45 87.8) (end 70.6 87.8) (width 0.2) (layer B.Cu) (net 6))
 (segment (start 46.6 59.4) (end 46.6 86.2) (width 0.2) (layer B.Cu) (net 6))
 (segment (start 36.6 49.4) (end 36.6 96.2) (width 0.2) (layer B.Cu) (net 6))
 (segment (start 71.8 56.2) (end 43.4 56.2) (width 0.2) (layer B.Cu) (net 6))
 (segment (start 68.6 59.4) (end 46.6 59.4) (width 0.2) (layer B.Cu) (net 6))
 (segment (start 47 59.8) (end 47 85.8) (width 0.2) (layer B.Cu) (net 6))
 (segment (start 44.2 88.6) (end 71.4 88.6) (width 0.2) (layer B.Cu) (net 6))
 (segment (start 69 59) (end 46.2 59) (width 0.2) (layer B.Cu) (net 6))
 (segment (start 79.8 48.2) (end 35.4 48.2) (width 0.2) (layer B.Cu) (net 6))
 (segment (start 58.8 85.4) (end 68.2 85.4) (width 0.2) (layer B.Cu) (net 6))
 (segment (start 78.6 49.4) (end 36.6 49.4) (width 0.2) (layer B.Cu) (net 6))
 (segment (start 73.8 54.2) (end 41.4 54.2) (width 0.2) (layer B.Cu) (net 6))
 (segment (start 70.6 87.8) (end 70.6 57.4) (width 0.2) (layer B.Cu) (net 6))
 (segment (start 68.2 59.8) (end 47 59.8) (width 0.2) (layer B.Cu) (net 6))
 (segment (start 43 55.8) (end 43 89.8) (width 0.2) (layer B.Cu) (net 6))
 (segment (start 47 85.8) (end 68.6 85.8) (width 0.2) (layer B.Cu) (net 6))
 (segment (start 37.8 95) (end 77.8 95) (width 0.2) (layer B.Cu) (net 6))
 (segment (start 68.2 85.4) (end 68.2 59.8) (width 0.2) (layer B.Cu) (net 6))
 (segment (start 36.2 96.6) (end 79.4 96.6) (width 0.2) (layer B.Cu) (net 6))
 (segment (start 72.2 89.4) (end 72.2 55.8) (width 0.2) (layer B.Cu) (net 6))
 (segment (start 69.4 86.6) (end 69.4 58.6) (width 0.2) (layer B.Cu) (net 6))
 (segment (start 71.4 88.6) (end 71.4 56.6) (width 0.2) (layer B.Cu) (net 6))
 (segment (start 45.4 58.2) (end 45.4 87.4) (width 0.2) (layer B.Cu) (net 6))
 (segment (start 43 89.8) (end 72.6 89.8) (width 0.2) (layer B.Cu) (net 6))
 (segment (start 69.4 58.6) (end 45.8 58.6) (width 0.2) (layer B.Cu) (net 6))
 (segment (start 45.8 58.6) (end 45.8 87) (width 0.2) (layer B.Cu) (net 6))
 (segment (start 45.8 87) (end 69.8 87) (width 0.2) (layer B.Cu) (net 6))
 (segment (start 77.8 95) (end 77.8 50.2) (width 0.2) (layer B.Cu) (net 6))
 (segment (start 43.4 89.4) (end 72.2 89.4) (width 0.2) (layer B.Cu) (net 6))
 (segment (start 69.8 58.2) (end 45.4 58.2) (width 0.2) (layer B.Cu) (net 6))
 (segment (start 68.6 85.8) (end 68.6 59.4) (width 0.2) (layer B.Cu) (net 6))
 (segment (start 35.4 48.2) (end 35.4 97.4) (width 0.2) (layer B.Cu) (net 6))
 (segment (start 44.6 88.2) (end 71 88.2) (width 0.2) (layer B.Cu) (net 6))
 (segment (start 45.4 87.4) (end 70.2 87.4) (width 0.2) (layer B.Cu) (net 6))
 (segment (start 77.4 50.6) (end 37.8 50.6) (width 0.2) (layer B.Cu) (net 6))
 (segment (start 70.2 87.4) (end 70.2 57.8) (width 0.2) (layer B.Cu) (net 6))
 (segment (start 70.6 57.4) (end 44.6 57.4) (width 0.2) (layer B.Cu) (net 6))
 (segment (start 70.2 57.8) (end 45 57.8) (width 0.2) (layer B.Cu) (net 6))
 (segment (start 79 49) (end 36.2 49) (width 0.2) (layer B.Cu) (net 6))
 (segment (start 44.6 57.4) (end 44.6 88.2) (width 0.2) (layer B.Cu) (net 6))
 (segment (start 45 57.8) (end 45 87.8) (width 0.2) (layer B.Cu) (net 6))
 (segment (start 41.4 54.2) (end 41.4 91.4) (width 0.2) (layer B.Cu) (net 6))
 (segment (start 41.4 91.4) (end 74.2 91.4) (width 0.2) (layer B.Cu) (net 6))
 (segment (start 74.2 91.4) (end 74.2 53.8) (width 0.2) (layer B.Cu) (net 6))
 (segment (start 74.2 53.8) (end 41 53.8) (width 0.2) (layer B.Cu) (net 6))
 (segment (start 41 53.8) (end 41 91.8) (width 0.2) (layer B.Cu) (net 6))
 (segment (start 41 91.8) (end 74.6 91.8) (width 0.2) (layer B.Cu) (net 6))
 (segment (start 74.6 91.8) (end 74.6 53.4) (width 0.2) (layer B.Cu) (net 6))
 (segment (start 74.6 53.4) (end 40.6 53.4) (width 0.2) (layer B.Cu) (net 6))
 (segment (start 40.6 53.4) (end 40.6 92.2) (width 0.2) (layer B.Cu) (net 6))
 (segment (start 40.6 92.2) (end 75 92.2) (width 0.2) (layer B.Cu) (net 6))
 (segment (start 75 92.2) (end 75 53) (width 0.2) (layer B.Cu) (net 6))
 (segment (start 75 53) (end 40.2 53) (width 0.2) (layer B.Cu) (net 6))
 (segment (start 40.2 53) (end 40.2 92.6) (width 0.2) (layer B.Cu) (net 6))
 (segment (start 40.2 92.6) (end 75.4 92.6) (width 0.2) (layer B.Cu) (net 6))
 (segment (start 75.4 92.6) (end 75.4 52.6) (width 0.2) (layer B.Cu) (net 6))
 (segment (start 75.4 52.6) (end 39.8 52.6) (width 0.2) (layer B.Cu) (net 6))
 (segment (start 39.8 52.6) (end 39.8 93) (width 0.2) (layer B.Cu) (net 6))
 (segment (start 39.8 93) (end 75.8 93) (width 0.2) (layer B.Cu) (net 6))
 (segment (start 75.8 93) (end 75.8 52.2) (width 0.2) (layer B.Cu) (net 6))
 (segment (start 75.8 52.2) (end 39.4 52.2) (width 0.2) (layer B.Cu) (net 6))
 (segment (start 39.4 52.2) (end 39.4 93.4) (width 0.2) (layer B.Cu) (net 6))
 (segment (start 39.4 93.4) (end 76.2 93.4) (width 0.2) (layer B.Cu) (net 6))
 (segment (start 76.2 93.4) (end 76.2 51.8) (width 0.2) (layer B.Cu) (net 6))
 (segment (start 76.2 51.8) (end 39 51.8) (width 0.2) (layer B.Cu) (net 6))
 (segment (start 39 51.8) (end 39 93.8) (width 0.2) (layer B.Cu) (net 6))
 (segment (start 39 93.8) (end 76.6 93.8) (width 0.2) (layer B.Cu) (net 6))
 (segment (start 76.6 93.8) (end 76.6 51.4) (width 0.2) (layer B.Cu) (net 6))
 (segment (start 76.6 51.4) (end 38.6 51.4) (width 0.2) (layer B.Cu) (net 6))
 (segment (start 38.6 51.4) (end 38.6 94.2) (width 0.2) (layer B.Cu) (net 6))
 (segment (start 38.6 94.2) (end 77 94.2) (width 0.2) (layer B.Cu) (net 6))
 (segment (start 77 94.2) (end 77 51) (width 0.2) (layer B.Cu) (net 6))
 (segment (start 77 51) (end 38.2 51) (width 0.2) (layer B.Cu) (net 6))
 (segment (start 38.2 94.6) (end 77.4 94.6) (width 0.2) (layer B.Cu) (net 6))
 (segment (start 77.4 94.6) (end 77.4 50.6) (width 0.2) (layer B.Cu) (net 6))
 (segment (start 37.8 50.6) (end 37.8 95) (width 0.2) (layer B.Cu) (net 6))
 (segment (start 77.8 50.2) (end 37.4 50.2) (width 0.2) (layer B.Cu) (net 6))
 (segment (start 37.4 95.4) (end 78.2 95.4) (width 0.2) (layer B.Cu) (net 6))
 (segment (start 78.2 95.4) (end 78.2 49.8) (width 0.2) (layer B.Cu) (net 6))
 (segment (start 78.2 49.8) (end 37 49.8) (width 0.2) (layer B.Cu) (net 6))
 (segment (start 37 49.8) (end 37 95.8) (width 0.2) (layer B.Cu) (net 6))
 (segment (start 37 95.8) (end 78.6 95.8) (width 0.2) (layer B.Cu) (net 6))
 (segment (start 78.6 95.8) (end 78.6 49.4) (width 0.2) (layer B.Cu) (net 6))
 (segment (start 36.6 96.2) (end 79 96.2) (width 0.2) (layer B.Cu) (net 6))
 (segment (start 79 96.2) (end 79 49) (width 0.2) (layer B.Cu) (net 6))
 (segment (start 36.2 49) (end 36.2 96.6) (width 0.2) (layer B.Cu) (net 6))
 (segment (start 79.4 96.6) (end 79.4 48.6) (width 0.2) (layer B.Cu) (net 6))
 (segment (start 79.4 48.6) (end 35.8 48.6) (width 0.2) (layer B.Cu) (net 6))
 (segment (start 35.8 48.6) (end 35.8 97) (width 0.2) (layer B.Cu) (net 6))
 (segment (start 35.8 97) (end 79.8 97) (width 0.2) (layer B.Cu) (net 6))
 (segment (start 79.8 97) (end 79.8 48.2) (width 0.2) (layer B.Cu) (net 6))
 (segment (start 35.4 97.4) (end 80.2 97.4) (width 0.2) (layer B.Cu) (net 6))
 (segment (start 80.2 47.8) (end 35 47.8) (width 0.2) (layer B.Cu) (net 6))
 (segment (start 35 47.8) (end 35 97.8) (width 0.2) (layer B.Cu) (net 6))
 (segment (start 80.6 97.8) (end 80.6 47.4) (width 0.2) (layer B.Cu) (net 6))
 (segment (start 80.6 47.4) (end 34.6 47.4) (width 0.2) (layer B.Cu) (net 6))
 (via (at 30.6 102.2) (size 0.3) (drill 0.2) (layers F.Cu B.Cu) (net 6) (status 1000000))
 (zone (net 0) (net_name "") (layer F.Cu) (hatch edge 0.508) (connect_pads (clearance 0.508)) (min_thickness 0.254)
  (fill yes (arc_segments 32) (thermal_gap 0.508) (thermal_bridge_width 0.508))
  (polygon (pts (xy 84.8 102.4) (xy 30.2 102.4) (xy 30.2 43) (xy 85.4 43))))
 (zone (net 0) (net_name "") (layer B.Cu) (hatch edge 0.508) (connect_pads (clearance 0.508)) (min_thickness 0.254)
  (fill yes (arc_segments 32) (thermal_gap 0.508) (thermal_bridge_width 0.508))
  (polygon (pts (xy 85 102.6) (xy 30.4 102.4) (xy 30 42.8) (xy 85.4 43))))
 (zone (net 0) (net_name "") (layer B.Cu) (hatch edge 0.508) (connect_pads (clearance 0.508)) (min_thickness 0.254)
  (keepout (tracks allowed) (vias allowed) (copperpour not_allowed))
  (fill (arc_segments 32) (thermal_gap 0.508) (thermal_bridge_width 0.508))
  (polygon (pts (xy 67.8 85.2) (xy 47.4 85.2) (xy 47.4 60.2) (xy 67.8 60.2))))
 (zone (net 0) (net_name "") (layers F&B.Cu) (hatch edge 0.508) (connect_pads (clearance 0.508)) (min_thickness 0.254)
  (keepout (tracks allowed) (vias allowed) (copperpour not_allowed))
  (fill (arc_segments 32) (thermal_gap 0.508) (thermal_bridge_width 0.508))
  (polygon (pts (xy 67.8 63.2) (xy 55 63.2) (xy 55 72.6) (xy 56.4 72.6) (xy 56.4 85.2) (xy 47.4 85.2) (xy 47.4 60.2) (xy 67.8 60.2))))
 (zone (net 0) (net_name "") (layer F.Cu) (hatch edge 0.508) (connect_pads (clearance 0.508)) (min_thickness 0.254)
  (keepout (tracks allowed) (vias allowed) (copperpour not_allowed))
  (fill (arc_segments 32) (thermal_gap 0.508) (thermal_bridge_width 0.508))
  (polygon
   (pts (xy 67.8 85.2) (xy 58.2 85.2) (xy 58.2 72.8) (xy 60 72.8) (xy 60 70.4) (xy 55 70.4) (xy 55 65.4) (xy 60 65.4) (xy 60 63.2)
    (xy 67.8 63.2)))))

